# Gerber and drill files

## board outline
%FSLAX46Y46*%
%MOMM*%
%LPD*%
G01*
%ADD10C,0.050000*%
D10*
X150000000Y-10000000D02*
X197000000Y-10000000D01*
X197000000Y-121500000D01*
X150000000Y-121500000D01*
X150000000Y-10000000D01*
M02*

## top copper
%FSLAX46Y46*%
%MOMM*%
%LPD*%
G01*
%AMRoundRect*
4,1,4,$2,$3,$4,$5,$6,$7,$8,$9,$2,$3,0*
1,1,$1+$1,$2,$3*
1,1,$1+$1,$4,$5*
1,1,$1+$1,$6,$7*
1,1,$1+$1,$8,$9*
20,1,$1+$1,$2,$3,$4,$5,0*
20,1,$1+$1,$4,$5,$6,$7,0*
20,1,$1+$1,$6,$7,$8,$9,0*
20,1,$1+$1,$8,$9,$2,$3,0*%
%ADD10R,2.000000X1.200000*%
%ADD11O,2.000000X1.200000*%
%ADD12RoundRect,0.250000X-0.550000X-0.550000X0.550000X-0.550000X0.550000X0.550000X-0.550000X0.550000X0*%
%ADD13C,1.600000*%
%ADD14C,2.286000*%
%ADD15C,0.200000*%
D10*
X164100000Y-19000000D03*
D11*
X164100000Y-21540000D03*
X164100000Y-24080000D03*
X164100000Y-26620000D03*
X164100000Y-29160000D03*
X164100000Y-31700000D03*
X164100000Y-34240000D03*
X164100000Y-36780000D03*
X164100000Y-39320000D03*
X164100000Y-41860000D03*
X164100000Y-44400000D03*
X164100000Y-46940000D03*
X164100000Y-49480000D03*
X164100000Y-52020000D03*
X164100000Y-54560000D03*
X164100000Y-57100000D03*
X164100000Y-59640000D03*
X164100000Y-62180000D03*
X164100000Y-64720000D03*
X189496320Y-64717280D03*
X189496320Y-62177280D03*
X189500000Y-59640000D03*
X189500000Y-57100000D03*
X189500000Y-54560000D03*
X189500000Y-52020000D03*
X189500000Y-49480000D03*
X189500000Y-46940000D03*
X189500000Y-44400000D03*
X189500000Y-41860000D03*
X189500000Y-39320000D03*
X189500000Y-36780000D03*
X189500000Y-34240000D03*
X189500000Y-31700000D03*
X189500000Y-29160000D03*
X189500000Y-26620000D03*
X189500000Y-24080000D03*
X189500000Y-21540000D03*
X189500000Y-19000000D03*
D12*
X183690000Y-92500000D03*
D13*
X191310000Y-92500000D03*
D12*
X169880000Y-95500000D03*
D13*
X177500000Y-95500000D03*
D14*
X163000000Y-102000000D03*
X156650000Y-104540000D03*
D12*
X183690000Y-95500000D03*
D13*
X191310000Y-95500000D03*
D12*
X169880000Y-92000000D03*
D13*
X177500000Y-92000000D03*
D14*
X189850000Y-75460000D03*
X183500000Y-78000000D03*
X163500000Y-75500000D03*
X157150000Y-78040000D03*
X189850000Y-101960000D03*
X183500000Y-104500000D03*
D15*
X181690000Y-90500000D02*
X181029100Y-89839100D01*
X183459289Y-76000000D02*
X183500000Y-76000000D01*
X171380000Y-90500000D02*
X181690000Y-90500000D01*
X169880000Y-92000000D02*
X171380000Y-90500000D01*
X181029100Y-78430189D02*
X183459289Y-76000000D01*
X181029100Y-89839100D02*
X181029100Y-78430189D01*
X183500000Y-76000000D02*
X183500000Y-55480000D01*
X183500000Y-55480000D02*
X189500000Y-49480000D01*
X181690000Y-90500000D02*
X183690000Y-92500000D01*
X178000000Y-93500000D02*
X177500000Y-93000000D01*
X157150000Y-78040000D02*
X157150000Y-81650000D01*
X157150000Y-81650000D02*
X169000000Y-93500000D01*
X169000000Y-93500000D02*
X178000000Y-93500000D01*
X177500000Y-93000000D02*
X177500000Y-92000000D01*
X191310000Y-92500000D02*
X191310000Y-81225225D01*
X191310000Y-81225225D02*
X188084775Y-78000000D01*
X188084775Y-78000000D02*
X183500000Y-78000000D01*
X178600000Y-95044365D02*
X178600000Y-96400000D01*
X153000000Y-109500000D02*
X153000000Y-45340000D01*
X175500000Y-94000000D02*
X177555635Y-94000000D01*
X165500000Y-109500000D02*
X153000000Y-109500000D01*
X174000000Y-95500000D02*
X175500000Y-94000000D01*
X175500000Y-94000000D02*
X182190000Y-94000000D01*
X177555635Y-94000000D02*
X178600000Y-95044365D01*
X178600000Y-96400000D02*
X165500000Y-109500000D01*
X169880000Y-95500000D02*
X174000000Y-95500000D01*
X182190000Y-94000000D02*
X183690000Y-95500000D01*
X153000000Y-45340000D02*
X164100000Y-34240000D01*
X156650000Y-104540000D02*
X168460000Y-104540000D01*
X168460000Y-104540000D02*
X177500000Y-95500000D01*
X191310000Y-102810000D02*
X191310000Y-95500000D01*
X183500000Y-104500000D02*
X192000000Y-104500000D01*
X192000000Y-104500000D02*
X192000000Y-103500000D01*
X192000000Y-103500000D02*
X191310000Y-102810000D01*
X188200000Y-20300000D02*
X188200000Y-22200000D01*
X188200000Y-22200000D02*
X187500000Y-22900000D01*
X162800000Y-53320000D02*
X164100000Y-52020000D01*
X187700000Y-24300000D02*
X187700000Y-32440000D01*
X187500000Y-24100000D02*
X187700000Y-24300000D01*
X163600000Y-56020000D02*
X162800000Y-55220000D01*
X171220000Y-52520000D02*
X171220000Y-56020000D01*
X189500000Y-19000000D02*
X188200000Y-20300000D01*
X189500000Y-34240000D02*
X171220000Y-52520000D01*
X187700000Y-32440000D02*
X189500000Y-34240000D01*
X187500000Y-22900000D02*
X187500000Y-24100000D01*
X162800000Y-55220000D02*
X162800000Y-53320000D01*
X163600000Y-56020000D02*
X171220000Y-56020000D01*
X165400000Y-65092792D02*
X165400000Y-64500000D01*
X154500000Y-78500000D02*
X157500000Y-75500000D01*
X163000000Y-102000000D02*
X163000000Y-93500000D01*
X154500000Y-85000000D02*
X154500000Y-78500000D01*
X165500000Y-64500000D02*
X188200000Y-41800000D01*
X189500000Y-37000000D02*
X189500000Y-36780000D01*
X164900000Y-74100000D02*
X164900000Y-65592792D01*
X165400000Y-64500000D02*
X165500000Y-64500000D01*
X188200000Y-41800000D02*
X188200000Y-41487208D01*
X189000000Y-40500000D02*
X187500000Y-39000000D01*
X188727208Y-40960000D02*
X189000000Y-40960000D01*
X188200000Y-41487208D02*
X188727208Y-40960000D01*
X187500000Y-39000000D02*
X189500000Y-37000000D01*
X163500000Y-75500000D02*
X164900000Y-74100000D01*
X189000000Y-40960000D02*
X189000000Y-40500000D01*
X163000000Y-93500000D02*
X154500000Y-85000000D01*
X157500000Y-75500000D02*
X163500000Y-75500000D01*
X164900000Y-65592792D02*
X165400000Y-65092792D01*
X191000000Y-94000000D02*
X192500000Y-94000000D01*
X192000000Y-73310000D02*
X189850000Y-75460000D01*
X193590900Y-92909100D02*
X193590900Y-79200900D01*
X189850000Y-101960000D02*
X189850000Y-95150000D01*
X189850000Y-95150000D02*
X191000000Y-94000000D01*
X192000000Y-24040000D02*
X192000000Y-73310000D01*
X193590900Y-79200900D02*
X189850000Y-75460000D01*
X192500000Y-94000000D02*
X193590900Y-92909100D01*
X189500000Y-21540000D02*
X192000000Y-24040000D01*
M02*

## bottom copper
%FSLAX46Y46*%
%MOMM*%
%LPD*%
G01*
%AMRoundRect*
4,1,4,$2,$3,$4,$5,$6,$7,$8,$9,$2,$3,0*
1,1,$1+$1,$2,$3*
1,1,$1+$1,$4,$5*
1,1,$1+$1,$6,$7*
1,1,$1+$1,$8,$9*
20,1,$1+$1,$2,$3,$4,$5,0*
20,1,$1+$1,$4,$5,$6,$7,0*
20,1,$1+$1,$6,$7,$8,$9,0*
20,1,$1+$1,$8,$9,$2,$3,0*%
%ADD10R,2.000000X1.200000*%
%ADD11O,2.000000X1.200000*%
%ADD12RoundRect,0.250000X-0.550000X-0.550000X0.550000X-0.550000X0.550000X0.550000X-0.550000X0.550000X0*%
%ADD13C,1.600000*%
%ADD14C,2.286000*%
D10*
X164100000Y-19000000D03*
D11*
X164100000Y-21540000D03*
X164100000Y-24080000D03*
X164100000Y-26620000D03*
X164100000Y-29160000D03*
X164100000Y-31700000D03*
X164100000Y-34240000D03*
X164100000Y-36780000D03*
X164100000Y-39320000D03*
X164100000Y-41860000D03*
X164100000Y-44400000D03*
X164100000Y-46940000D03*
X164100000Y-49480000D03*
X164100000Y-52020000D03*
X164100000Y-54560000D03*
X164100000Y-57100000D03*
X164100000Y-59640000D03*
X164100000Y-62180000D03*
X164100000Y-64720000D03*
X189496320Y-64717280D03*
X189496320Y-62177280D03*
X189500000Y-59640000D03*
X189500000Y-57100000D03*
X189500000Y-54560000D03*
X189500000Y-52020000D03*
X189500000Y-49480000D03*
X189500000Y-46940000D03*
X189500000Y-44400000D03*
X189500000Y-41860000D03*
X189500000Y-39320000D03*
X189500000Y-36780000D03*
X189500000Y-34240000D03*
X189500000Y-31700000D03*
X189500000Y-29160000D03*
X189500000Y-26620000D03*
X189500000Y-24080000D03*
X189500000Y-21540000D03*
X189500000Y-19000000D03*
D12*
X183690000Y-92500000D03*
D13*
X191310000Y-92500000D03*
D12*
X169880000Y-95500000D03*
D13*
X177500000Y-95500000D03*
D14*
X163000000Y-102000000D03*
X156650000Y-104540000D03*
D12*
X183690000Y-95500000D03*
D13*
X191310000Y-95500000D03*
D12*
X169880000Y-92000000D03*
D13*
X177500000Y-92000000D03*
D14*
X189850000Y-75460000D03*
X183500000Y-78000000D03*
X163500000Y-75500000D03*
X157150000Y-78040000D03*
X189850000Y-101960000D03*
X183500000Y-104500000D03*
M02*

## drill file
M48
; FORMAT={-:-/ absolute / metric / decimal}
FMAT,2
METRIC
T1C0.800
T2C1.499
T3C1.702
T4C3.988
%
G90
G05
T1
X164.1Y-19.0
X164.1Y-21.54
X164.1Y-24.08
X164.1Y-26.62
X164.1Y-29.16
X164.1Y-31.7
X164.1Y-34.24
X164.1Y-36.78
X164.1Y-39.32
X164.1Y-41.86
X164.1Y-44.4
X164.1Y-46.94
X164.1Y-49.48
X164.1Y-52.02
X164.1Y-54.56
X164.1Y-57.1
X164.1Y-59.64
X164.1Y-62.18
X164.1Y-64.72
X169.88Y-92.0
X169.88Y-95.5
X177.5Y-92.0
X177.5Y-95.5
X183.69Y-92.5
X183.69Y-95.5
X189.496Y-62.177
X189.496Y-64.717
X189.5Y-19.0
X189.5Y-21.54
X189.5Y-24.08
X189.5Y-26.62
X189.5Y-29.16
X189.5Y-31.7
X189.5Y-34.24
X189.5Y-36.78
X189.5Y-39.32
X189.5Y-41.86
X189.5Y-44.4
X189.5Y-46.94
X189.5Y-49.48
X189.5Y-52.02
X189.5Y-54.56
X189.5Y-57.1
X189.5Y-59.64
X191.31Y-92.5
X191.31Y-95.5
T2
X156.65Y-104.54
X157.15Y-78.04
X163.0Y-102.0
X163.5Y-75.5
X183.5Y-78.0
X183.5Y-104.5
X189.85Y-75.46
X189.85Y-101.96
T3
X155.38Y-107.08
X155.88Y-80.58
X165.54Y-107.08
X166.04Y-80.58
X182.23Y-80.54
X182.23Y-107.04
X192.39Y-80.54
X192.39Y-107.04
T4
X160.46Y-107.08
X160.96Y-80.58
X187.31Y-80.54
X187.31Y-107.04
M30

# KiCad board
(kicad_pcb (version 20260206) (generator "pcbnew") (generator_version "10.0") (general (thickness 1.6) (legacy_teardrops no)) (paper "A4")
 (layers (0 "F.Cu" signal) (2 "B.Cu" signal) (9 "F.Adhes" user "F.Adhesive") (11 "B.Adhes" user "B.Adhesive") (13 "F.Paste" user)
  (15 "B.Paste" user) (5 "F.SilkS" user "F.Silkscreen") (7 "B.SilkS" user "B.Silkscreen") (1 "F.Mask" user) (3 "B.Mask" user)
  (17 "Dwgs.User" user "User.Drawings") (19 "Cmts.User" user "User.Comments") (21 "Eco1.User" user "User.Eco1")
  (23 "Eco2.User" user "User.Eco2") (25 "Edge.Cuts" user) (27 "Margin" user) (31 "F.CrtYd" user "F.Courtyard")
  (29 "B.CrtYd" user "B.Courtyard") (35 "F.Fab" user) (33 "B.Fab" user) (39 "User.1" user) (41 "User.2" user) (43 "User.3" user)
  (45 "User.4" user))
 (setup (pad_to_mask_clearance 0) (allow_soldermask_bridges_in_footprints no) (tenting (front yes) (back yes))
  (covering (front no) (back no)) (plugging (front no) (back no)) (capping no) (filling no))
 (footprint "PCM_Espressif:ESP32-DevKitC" (layer "F.Cu") (at 164.1 19)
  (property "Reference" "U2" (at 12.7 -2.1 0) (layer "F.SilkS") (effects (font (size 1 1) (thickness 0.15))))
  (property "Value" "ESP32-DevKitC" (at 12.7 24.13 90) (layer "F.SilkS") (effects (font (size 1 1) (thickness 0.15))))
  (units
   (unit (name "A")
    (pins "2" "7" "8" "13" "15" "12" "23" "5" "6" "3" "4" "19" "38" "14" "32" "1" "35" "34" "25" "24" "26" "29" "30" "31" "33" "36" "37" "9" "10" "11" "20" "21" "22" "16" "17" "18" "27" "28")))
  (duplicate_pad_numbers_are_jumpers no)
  (pad "1" thru_hole rect (at 0 0 270) (size 1.2 2) (drill 0.8) (layers "*.Cu" "*.Mask") (remove_unused_layers no) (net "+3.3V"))
  (pad "2" thru_hole oval (at 0 2.54 270) (size 1.2 2) (drill 0.8) (layers "*.Cu" "*.Mask") (remove_unused_layers no)
   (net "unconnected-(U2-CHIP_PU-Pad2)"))
  (pad "3" thru_hole oval (at 0 5.08 270) (size 1.2 2) (drill 0.8) (layers "*.Cu" "*.Mask") (remove_unused_layers no)
   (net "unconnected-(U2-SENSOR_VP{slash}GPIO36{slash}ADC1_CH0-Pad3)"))
  (pad "4" thru_hole oval (at 0 7.62 270) (size 1.2 2) (drill 0.8) (layers "*.Cu" "*.Mask") (remove_unused_layers no)
   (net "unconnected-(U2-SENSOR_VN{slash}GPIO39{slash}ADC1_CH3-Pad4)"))
  (pad "5" thru_hole oval (at 0 10.16 270) (size 1.2 2) (drill 0.8) (layers "*.Cu" "*.Mask") (remove_unused_layers no)
   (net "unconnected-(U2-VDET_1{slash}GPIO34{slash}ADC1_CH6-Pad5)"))
  (pad "6" thru_hole oval (at 0 12.7 270) (size 1.2 2) (drill 0.8) (layers "*.Cu" "*.Mask") (remove_unused_layers no)
   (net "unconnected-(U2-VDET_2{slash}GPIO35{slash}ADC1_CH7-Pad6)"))
  (pad "7" thru_hole oval (at 0 15.24 270) (size 1.2 2) (drill 0.8) (layers "*.Cu" "*.Mask") (remove_unused_layers no) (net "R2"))
  (pad "8" thru_hole oval (at 0 17.78 270) (size 1.2 2) (drill 0.8) (layers "*.Cu" "*.Mask") (remove_unused_layers no)
   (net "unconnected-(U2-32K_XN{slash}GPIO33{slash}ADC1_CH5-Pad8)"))
  (pad "9" thru_hole oval (at 0 20.32 270) (size 1.2 2) (drill 0.8) (layers "*.Cu" "*.Mask") (remove_unused_layers no)
   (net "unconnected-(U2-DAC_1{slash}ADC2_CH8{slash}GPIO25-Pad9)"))
  (pad "10" thru_hole oval (at 0 22.86 270) (size 1.2 2) (drill 0.8) (layers "*.Cu" "*.Mask") (remove_unused_layers no)
   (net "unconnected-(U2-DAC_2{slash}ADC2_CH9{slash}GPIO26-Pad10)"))
  (pad "11" thru_hole oval (at 0 25.4 270) (size 1.2 2) (drill 0.8) (layers "*.Cu" "*.Mask") (remove_unused_layers no)
   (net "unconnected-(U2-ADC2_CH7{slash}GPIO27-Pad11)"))
  (pad "12" thru_hole oval (at 0 27.94 270) (size 1.2 2) (drill 0.8) (layers "*.Cu" "*.Mask") (remove_unused_layers no)
   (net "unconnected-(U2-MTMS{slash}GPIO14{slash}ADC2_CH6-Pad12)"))
  (pad "13" thru_hole oval (at 0 30.48 270) (size 1.2 2) (drill 0.8) (layers "*.Cu" "*.Mask") (remove_unused_layers no)
   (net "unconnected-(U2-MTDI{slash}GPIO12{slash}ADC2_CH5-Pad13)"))
  (pad "14" thru_hole oval (at 0 33.02 270) (size 1.2 2) (drill 0.8) (layers "*.Cu" "*.Mask") (remove_unused_layers no) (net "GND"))
  (pad "15" thru_hole oval (at 0 35.56 270) (size 1.2 2) (drill 0.8) (layers "*.Cu" "*.Mask") (remove_unused_layers no)
   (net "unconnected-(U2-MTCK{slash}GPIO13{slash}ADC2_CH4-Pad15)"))
  (pad "16" thru_hole oval (at 0 38.1 270) (size 1.2 2) (drill 0.8) (layers "*.Cu" "*.Mask") (remove_unused_layers no)
   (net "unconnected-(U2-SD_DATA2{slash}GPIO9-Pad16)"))
  (pad "17" thru_hole oval (at 0 40.64 270) (size 1.2 2) (drill 0.8) (layers "*.Cu" "*.Mask") (remove_unused_layers no)
   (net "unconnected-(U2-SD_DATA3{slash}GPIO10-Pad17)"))
  (pad "18" thru_hole oval (at 0 43.18 270) (size 1.2 2) (drill 0.8) (layers "*.Cu" "*.Mask") (remove_unused_layers no)
   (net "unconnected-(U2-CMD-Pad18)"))
  (pad "19" thru_hole oval (at 0 45.72 270) (size 1.2 2) (drill 0.8) (layers "*.Cu" "*.Mask") (remove_unused_layers no)
   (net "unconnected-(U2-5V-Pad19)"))
  (pad "20" thru_hole oval (at 25.39632 45.71728 270) (size 1.2 2) (drill 0.8) (layers "*.Cu" "*.Mask") (remove_unused_layers no)
   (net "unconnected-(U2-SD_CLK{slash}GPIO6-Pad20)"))
  (pad "21" thru_hole oval (at 25.39632 43.17728 270) (size 1.2 2) (drill 0.8) (layers "*.Cu" "*.Mask") (remove_unused_layers no)
   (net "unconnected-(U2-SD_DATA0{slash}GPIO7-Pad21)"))
  (pad "22" thru_hole oval (at 25.4 40.64 270) (size 1.2 2) (drill 0.8) (layers "*.Cu" "*.Mask") (remove_unused_layers no)
   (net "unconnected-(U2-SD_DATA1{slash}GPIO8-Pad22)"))
  (pad "23" thru_hole oval (at 25.4 38.1 270) (size 1.2 2) (drill 0.8) (layers "*.Cu" "*.Mask") (remove_unused_layers no)
   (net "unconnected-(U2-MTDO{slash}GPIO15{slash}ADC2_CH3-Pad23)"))
  (pad "24" thru_hole oval (at 25.4 35.56 270) (size 1.2 2) (drill 0.8) (layers "*.Cu" "*.Mask") (remove_unused_layers no)
   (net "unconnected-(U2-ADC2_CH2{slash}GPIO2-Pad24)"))
  (pad "25" thru_hole oval (at 25.4 33.02 270) (size 1.2 2) (drill 0.8) (layers "*.Cu" "*.Mask") (remove_unused_layers no)
   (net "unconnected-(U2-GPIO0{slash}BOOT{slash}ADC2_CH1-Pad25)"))
  (pad "26" thru_hole oval (at 25.4 30.48 270) (size 1.2 2) (drill 0.8) (layers "*.Cu" "*.Mask") (remove_unused_layers no) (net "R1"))
  (pad "27" thru_hole oval (at 25.4 27.94 270) (size 1.2 2) (drill 0.8) (layers "*.Cu" "*.Mask") (remove_unused_layers no)
   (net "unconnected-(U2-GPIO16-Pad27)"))
  (pad "28" thru_hole oval (at 25.4 25.4 270) (size 1.2 2) (drill 0.8) (layers "*.Cu" "*.Mask") (remove_unused_layers no)
   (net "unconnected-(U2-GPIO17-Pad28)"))
  (pad "29" thru_hole oval (at 25.4 22.86 270) (size 1.2 2) (drill 0.8) (layers "*.Cu" "*.Mask") (remove_unused_layers no)
   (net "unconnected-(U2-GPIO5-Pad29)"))
  (pad "30" thru_hole oval (at 25.4 20.32 270) (size 1.2 2) (drill 0.8) (layers "*.Cu" "*.Mask") (remove_unused_layers no)
   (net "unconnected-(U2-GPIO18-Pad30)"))
  (pad "31" thru_hole oval (at 25.4 17.78 270) (size 1.2 2) (drill 0.8) (layers "*.Cu" "*.Mask") (remove_unused_layers no) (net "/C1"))
  (pad "32" thru_hole oval (at 25.4 15.24 270) (size 1.2 2) (drill 0.8) (layers "*.Cu" "*.Mask") (remove_unused_layers no) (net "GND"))
  (pad "33" thru_hole oval (at 25.4 12.7 270) (size 1.2 2) (drill 0.8) (layers "*.Cu" "*.Mask") (remove_unused_layers no)
   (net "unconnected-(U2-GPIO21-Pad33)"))
  (pad "34" thru_hole oval (at 25.4 10.16 270) (size 1.2 2) (drill 0.8) (layers "*.Cu" "*.Mask") (remove_unused_layers no)
   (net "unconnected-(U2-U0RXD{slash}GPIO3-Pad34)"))
  (pad "35" thru_hole oval (at 25.4 7.62 270) (size 1.2 2) (drill 0.8) (layers "*.Cu" "*.Mask") (remove_unused_layers no)
   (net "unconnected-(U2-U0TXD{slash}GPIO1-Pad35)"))
  (pad "36" thru_hole oval (at 25.4 5.08 270) (size 1.2 2) (drill 0.8) (layers "*.Cu" "*.Mask") (remove_unused_layers no)
   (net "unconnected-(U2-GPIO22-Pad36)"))
  (pad "37" thru_hole oval (at 25.4 2.54 270) (size 1.2 2) (drill 0.8) (layers "*.Cu" "*.Mask") (remove_unused_layers no) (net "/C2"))
  (pad "38" thru_hole oval (at 25.4 0 270) (size 1.2 2) (drill 0.8) (layers "*.Cu" "*.Mask") (remove_unused_layers no) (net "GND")))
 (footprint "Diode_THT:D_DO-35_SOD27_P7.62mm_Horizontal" (layer "F.Cu") (at 183.69 92.5)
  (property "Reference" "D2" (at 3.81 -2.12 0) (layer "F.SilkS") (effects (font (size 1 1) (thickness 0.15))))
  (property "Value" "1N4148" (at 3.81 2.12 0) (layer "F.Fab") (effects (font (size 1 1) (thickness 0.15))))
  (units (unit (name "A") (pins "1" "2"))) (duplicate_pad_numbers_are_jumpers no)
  (pad "1" thru_hole roundrect (at 0 0) (size 1.6 1.6) (drill 0.8) (layers "*.Cu" "*.Mask") (remove_unused_layers no)
   (roundrect_rratio 0.15625) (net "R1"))
  (pad "2" thru_hole circle (at 7.62 0) (size 1.6 1.6) (drill 0.8) (layers "*.Cu" "*.Mask") (remove_unused_layers no) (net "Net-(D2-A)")))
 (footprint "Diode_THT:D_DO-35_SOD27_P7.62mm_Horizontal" (layer "F.Cu") (at 169.88 95.5)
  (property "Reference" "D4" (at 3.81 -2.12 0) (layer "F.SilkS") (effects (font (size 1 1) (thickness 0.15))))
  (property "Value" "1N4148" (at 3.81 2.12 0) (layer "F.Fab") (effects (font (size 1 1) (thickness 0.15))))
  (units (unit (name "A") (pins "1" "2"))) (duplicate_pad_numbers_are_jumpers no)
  (pad "1" thru_hole roundrect (at 0 0) (size 1.6 1.6) (drill 0.8) (layers "*.Cu" "*.Mask") (remove_unused_layers no)
   (roundrect_rratio 0.15625) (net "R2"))
  (pad "2" thru_hole circle (at 7.62 0) (size 1.6 1.6) (drill 0.8) (layers "*.Cu" "*.Mask") (remove_unused_layers no) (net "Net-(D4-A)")))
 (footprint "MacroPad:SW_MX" (layer "F.Cu") (at 160.46 107.08)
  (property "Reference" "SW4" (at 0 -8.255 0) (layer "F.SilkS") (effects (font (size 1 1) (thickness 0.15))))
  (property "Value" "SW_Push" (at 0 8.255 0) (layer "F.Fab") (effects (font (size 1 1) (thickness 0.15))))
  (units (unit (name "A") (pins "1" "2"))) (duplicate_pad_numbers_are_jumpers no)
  (pad "" np_thru_hole circle (at -5.08 0) (size 1.7018 1.7018) (drill 1.7018) (layers "*.Cu" "*.Mask"))
  (pad "" np_thru_hole circle (at 0 0) (size 3.9878 3.9878) (drill 3.9878) (layers "*.Cu" "*.Mask"))
  (pad "" np_thru_hole circle (at 5.08 0) (size 1.7018 1.7018) (drill 1.7018) (layers "*.Cu" "*.Mask"))
  (pad "1" thru_hole circle (at 2.54 -5.08) (size 2.286 2.286) (drill 1.4986) (layers "*.Cu" "*.Mask") (remove_unused_layers no) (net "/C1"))
  (pad "2" thru_hole circle (at -3.81 -2.54) (size 2.286 2.286) (drill 1.4986) (layers "*.Cu" "*.Mask") (remove_unused_layers no)
   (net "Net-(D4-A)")))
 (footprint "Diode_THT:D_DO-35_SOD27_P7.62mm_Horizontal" (layer "F.Cu") (at 183.69 95.5)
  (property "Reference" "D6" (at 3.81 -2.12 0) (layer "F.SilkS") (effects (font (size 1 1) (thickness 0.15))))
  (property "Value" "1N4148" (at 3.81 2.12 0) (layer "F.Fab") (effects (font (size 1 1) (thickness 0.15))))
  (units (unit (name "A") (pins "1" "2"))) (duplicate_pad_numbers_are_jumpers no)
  (pad "1" thru_hole roundrect (at 0 0) (size 1.6 1.6) (drill 0.8) (layers "*.Cu" "*.Mask") (remove_unused_layers no)
   (roundrect_rratio 0.15625) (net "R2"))
  (pad "2" thru_hole circle (at 7.62 0) (size 1.6 1.6) (drill 0.8) (layers "*.Cu" "*.Mask") (remove_unused_layers no) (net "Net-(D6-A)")))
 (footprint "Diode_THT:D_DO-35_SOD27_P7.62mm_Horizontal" (layer "F.Cu") (at 169.88 92)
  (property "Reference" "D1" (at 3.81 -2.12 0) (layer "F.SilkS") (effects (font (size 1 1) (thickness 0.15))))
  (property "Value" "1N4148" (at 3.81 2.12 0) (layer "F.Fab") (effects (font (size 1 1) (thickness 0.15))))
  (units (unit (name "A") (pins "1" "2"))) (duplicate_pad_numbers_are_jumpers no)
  (pad "1" thru_hole roundrect (at 0 0) (size 1.6 1.6) (drill 0.8) (layers "*.Cu" "*.Mask") (remove_unused_layers no)
   (roundrect_rratio 0.15625) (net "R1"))
  (pad "2" thru_hole circle (at 7.62 0) (size 1.6 1.6) (drill 0.8) (layers "*.Cu" "*.Mask") (remove_unused_layers no) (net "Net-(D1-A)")))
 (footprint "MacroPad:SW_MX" (layer "F.Cu") (at 187.31 80.54)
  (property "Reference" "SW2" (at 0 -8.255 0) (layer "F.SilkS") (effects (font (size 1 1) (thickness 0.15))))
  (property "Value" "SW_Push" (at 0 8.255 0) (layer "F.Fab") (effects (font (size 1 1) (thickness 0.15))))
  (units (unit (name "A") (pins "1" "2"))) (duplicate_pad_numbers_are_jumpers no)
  (pad "" np_thru_hole circle (at -5.08 0) (size 1.7018 1.7018) (drill 1.7018) (layers "*.Cu" "*.Mask"))
  (pad "" np_thru_hole circle (at 0 0) (size 3.9878 3.9878) (drill 3.9878) (layers "*.Cu" "*.Mask"))
  (pad "" np_thru_hole circle (at 5.08 0) (size 1.7018 1.7018) (drill 1.7018) (layers "*.Cu" "*.Mask"))
  (pad "1" thru_hole circle (at 2.54 -5.08) (size 2.286 2.286) (drill 1.4986) (layers "*.Cu" "*.Mask") (remove_unused_layers no) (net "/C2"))
  (pad "2" thru_hole circle (at -3.81 -2.54) (size 2.286 2.286) (drill 1.4986) (layers "*.Cu" "*.Mask") (remove_unused_layers no)
   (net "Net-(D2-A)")))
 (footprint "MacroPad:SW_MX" (layer "F.Cu") (at 160.96 80.58)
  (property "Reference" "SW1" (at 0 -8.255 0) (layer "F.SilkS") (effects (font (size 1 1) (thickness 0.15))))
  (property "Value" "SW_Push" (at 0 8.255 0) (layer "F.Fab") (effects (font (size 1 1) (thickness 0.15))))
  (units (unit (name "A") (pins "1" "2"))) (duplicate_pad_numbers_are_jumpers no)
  (pad "" np_thru_hole circle (at -5.08 0) (size 1.7018 1.7018) (drill 1.7018) (layers "*.Cu" "*.Mask"))
  (pad "" np_thru_hole circle (at 0 0) (size 3.9878 3.9878) (drill 3.9878) (layers "*.Cu" "*.Mask"))
  (pad "" np_thru_hole circle (at 5.08 0) (size 1.7018 1.7018) (drill 1.7018) (layers "*.Cu" "*.Mask"))
  (pad "1" thru_hole circle (at 2.54 -5.08) (size 2.286 2.286) (drill 1.4986) (layers "*.Cu" "*.Mask") (remove_unused_layers no) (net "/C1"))
  (pad "2" thru_hole circle (at -3.81 -2.54) (size 2.286 2.286) (drill 1.4986) (layers "*.Cu" "*.Mask") (remove_unused_layers no)
   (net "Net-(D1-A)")))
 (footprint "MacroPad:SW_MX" (layer "F.Cu") (at 187.31 107.04)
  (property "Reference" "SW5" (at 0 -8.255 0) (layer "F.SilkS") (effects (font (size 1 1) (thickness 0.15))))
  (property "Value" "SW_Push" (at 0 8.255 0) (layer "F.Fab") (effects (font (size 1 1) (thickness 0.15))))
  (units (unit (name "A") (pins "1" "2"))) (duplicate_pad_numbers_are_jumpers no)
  (pad "" np_thru_hole circle (at -5.08 0) (size 1.7018 1.7018) (drill 1.7018) (layers "*.Cu" "*.Mask"))
  (pad "" np_thru_hole circle (at 0 0) (size 3.9878 3.9878) (drill 3.9878) (layers "*.Cu" "*.Mask"))
  (pad "" np_thru_hole circle (at 5.08 0) (size 1.7018 1.7018) (drill 1.7018) (layers "*.Cu" "*.Mask"))
  (pad "1" thru_hole circle (at 2.54 -5.08) (size 2.286 2.286) (drill 1.4986) (layers "*.Cu" "*.Mask") (remove_unused_layers no) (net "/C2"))
  (pad "2" thru_hole circle (at -3.81 -2.54) (size 2.286 2.286) (drill 1.4986) (layers "*.Cu" "*.Mask") (remove_unused_layers no)
   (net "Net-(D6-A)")))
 (gr_rect (start 150 10) (end 197 121.5) (stroke (width 0.05) (type default)) (fill no) (layer "Edge.Cuts"))
 (segment (start 181.69 90.5) (end 181.0291 89.8391) (width 0.2) (layer "F.Cu") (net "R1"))
 (segment (start 183.459289 76) (end 183.5 76) (width 0.2) (layer "F.Cu") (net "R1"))
 (segment (start 171.38 90.5) (end 181.69 90.5) (width 0.2) (layer "F.Cu") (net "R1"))
 (segment (start 169.88 92) (end 171.38 90.5) (width 0.2) (layer "F.Cu") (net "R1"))
 (segment (start 181.0291 78.430189) (end 183.459289 76) (width 0.2) (layer "F.Cu") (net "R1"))
 (segment (start 181.0291 89.8391) (end 181.0291 78.430189) (width 0.2) (layer "F.Cu") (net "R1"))
 (segment (start 183.5 76) (end 183.5 55.48) (width 0.2) (layer "F.Cu") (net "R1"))
 (segment (start 183.5 55.48) (end 189.5 49.48) (width 0.2) (layer "F.Cu") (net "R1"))
 (segment (start 181.69 90.5) (end 183.69 92.5) (width 0.2) (layer "F.Cu") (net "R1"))
 (segment (start 178 93.5) (end 177.5 93) (width 0.2) (layer "F.Cu") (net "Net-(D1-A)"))
 (segment (start 157.15 78.04) (end 157.15 81.65) (width 0.2) (layer "F.Cu") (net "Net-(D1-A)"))
 (segment (start 157.15 81.65) (end 169 93.5) (width 0.2) (layer "F.Cu") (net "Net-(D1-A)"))
 (segment (start 169 93.5) (end 178 93.5) (width 0.2) (layer "F.Cu") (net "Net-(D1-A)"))
 (segment (start 177.5 93) (end 177.5 92) (width 0.2) (layer "F.Cu") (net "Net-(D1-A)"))
 (segment (start 191.31 92.5) (end 191.31 81.225225) (width 0.2) (layer "F.Cu") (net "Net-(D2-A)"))
 (segment (start 191.31 81.225225) (end 188.084775 78) (width 0.2) (layer "F.Cu") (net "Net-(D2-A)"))
 (segment (start 188.084775 78) (end 183.5 78) (width 0.2) (layer "F.Cu") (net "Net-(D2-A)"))
 (segment (start 178.6 95.044365) (end 178.6 96.4) (width 0.2) (layer "F.Cu") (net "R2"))
 (segment (start 153 109.5) (end 153 45.34) (width 0.2) (layer "F.Cu") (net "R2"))
 (segment (start 175.5 94) (end 177.555635 94) (width 0.2) (layer "F.Cu") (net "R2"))
 (segment (start 165.5 109.5) (end 153 109.5) (width 0.2) (layer "F.Cu") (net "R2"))
 (segment (start 174 95.5) (end 175.5 94) (width 0.2) (layer "F.Cu") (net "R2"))
 (segment (start 175.5 94) (end 182.19 94) (width 0.2) (layer "F.Cu") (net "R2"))
 (segment (start 177.555635 94) (end 178.6 95.044365) (width 0.2) (layer "F.Cu") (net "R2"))
 (segment (start 178.6 96.4) (end 165.5 109.5) (width 0.2) (layer "F.Cu") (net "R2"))
 (segment (start 169.88 95.5) (end 174 95.5) (width 0.2) (layer "F.Cu") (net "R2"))
 (segment (start 182.19 94) (end 183.69 95.5) (width 0.2) (layer "F.Cu") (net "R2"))
 (segment (start 153 45.34) (end 164.1 34.24) (width 0.2) (layer "F.Cu") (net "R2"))
 (segment (start 156.65 104.54) (end 168.46 104.54) (width 0.2) (layer "F.Cu") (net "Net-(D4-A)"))
 (segment (start 168.46 104.54) (end 177.5 95.5) (width 0.2) (layer "F.Cu") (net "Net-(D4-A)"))
 (segment (start 191.31 102.81) (end 191.31 95.5) (width 0.2) (layer "F.Cu") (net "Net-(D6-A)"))
 (segment (start 183.5 104.5) (end 192 104.5) (width 0.2) (layer "F.Cu") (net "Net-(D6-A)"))
 (segment (start 192 104.5) (end 192 103.5) (width 0.2) (layer "F.Cu") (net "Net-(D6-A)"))
 (segment (start 192 103.5) (end 191.31 102.81) (width 0.2) (layer "F.Cu") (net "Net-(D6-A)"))
 (segment (start 188.2 20.3) (end 188.2 22.2) (width 0.2) (layer "F.Cu") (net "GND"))
 (segment (start 188.2 22.2) (end 187.5 22.9) (width 0.2) (layer "F.Cu") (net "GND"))
 (segment (start 162.8 53.32) (end 164.1 52.02) (width 0.2) (layer "F.Cu") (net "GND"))
 (segment (start 187.7 24.3) (end 187.7 32.44) (width 0.2) (layer "F.Cu") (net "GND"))
 (segment (start 187.5 24.1) (end 187.7 24.3) (width 0.2) (layer "F.Cu") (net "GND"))
 (segment (start 163.6 56.02) (end 162.8 55.22) (width 0.2) (layer "F.Cu") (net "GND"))
 (segment (start 171.22 52.52) (end 171.22 56.02) (width 0.2) (layer "F.Cu") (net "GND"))
 (segment (start 189.5 19) (end 188.2 20.3) (width 0.2) (layer "F.Cu") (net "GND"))
 (segment (start 189.5 34.24) (end 171.22 52.52) (width 0.2) (layer "F.Cu") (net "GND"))
 (segment (start 187.7 32.44) (end 189.5 34.24) (width 0.2) (layer "F.Cu") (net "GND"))
 (segment (start 187.5 22.9) (end 187.5 24.1) (width 0.2) (layer "F.Cu") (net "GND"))
 (segment (start 162.8 55.22) (end 162.8 53.32) (width 0.2) (layer "F.Cu") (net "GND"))
 (segment (start 163.6 56.02) (end 171.22 56.02) (width 0.2) (layer "F.Cu") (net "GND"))
 (segment (start 165.4 65.092792) (end 165.4 64.5) (width 0.2) (layer "F.Cu") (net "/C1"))
 (segment (start 154.5 78.5) (end 157.5 75.5) (width 0.2) (layer "F.Cu") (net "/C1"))
 (segment (start 163 102) (end 163 93.5) (width 0.2) (layer "F.Cu") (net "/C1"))
 (segment (start 154.5 85) (end 154.5 78.5) (width 0.2) (layer "F.Cu") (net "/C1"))
 (segment (start 165.5 64.5) (end 188.2 41.8) (width 0.2) (layer "F.Cu") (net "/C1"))
 (segment (start 189.5 37) (end 189.5 36.78) (width 0.2) (layer "F.Cu") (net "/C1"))
 (segment (start 164.9 74.1) (end 164.9 65.592792) (width 0.2) (layer "F.Cu") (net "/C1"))
 (segment (start 165.4 64.5) (end 165.5 64.5) (width 0.2) (layer "F.Cu") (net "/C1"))
 (segment (start 188.2 41.8) (end 188.2 41.487208) (width 0.2) (layer "F.Cu") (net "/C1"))
 (segment (start 189 40.5) (end 187.5 39) (width 0.2) (layer "F.Cu") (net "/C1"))
 (segment (start 188.727208 40.96) (end 189 40.96) (width 0.2) (layer "F.Cu") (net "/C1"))
 (segment (start 188.2 41.487208) (end 188.727208 40.96) (width 0.2) (layer "F.Cu") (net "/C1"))
 (segment (start 187.5 39) (end 189.5 37) (width 0.2) (layer "F.Cu") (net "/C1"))
 (segment (start 163.5 75.5) (end 164.9 74.1) (width 0.2) (layer "F.Cu") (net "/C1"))
 (segment (start 189 40.96) (end 189 40.5) (width 0.2) (layer "F.Cu") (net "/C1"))
 (segment (start 163 93.5) (end 154.5 85) (width 0.2) (layer "F.Cu") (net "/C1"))
 (segment (start 157.5 75.5) (end 163.5 75.5) (width 0.2) (layer "F.Cu") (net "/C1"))
 (segment (start 164.9 65.592792) (end 165.4 65.092792) (width 0.2) (layer "F.Cu") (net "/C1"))
 (segment (start 191 94) (end 192.5 94) (width 0.2) (layer "F.Cu") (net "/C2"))
 (segment (start 192 73.31) (end 189.85 75.46) (width 0.2) (layer "F.Cu") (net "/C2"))
 (segment (start 193.5909 92.9091) (end 193.5909 79.2009) (width 0.2) (layer "F.Cu") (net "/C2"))
 (segment (start 189.85 101.96) (end 189.85 95.15) (width 0.2) (layer "F.Cu") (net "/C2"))
 (segment (start 189.85 95.15) (end 191 94) (width 0.2) (layer "F.Cu") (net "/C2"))
 (segment (start 192 24.04) (end 192 73.31) (width 0.2) (layer "F.Cu") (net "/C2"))
 (segment (start 193.5909 79.2009) (end 189.85 75.46) (width 0.2) (layer "F.Cu") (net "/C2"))
 (segment (start 192.5 94) (end 193.5909 92.9091) (width 0.2) (layer "F.Cu") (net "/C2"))
 (segment (start 189.5 21.54) (end 192 24.04) (width 0.2) (layer "F.Cu") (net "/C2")))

